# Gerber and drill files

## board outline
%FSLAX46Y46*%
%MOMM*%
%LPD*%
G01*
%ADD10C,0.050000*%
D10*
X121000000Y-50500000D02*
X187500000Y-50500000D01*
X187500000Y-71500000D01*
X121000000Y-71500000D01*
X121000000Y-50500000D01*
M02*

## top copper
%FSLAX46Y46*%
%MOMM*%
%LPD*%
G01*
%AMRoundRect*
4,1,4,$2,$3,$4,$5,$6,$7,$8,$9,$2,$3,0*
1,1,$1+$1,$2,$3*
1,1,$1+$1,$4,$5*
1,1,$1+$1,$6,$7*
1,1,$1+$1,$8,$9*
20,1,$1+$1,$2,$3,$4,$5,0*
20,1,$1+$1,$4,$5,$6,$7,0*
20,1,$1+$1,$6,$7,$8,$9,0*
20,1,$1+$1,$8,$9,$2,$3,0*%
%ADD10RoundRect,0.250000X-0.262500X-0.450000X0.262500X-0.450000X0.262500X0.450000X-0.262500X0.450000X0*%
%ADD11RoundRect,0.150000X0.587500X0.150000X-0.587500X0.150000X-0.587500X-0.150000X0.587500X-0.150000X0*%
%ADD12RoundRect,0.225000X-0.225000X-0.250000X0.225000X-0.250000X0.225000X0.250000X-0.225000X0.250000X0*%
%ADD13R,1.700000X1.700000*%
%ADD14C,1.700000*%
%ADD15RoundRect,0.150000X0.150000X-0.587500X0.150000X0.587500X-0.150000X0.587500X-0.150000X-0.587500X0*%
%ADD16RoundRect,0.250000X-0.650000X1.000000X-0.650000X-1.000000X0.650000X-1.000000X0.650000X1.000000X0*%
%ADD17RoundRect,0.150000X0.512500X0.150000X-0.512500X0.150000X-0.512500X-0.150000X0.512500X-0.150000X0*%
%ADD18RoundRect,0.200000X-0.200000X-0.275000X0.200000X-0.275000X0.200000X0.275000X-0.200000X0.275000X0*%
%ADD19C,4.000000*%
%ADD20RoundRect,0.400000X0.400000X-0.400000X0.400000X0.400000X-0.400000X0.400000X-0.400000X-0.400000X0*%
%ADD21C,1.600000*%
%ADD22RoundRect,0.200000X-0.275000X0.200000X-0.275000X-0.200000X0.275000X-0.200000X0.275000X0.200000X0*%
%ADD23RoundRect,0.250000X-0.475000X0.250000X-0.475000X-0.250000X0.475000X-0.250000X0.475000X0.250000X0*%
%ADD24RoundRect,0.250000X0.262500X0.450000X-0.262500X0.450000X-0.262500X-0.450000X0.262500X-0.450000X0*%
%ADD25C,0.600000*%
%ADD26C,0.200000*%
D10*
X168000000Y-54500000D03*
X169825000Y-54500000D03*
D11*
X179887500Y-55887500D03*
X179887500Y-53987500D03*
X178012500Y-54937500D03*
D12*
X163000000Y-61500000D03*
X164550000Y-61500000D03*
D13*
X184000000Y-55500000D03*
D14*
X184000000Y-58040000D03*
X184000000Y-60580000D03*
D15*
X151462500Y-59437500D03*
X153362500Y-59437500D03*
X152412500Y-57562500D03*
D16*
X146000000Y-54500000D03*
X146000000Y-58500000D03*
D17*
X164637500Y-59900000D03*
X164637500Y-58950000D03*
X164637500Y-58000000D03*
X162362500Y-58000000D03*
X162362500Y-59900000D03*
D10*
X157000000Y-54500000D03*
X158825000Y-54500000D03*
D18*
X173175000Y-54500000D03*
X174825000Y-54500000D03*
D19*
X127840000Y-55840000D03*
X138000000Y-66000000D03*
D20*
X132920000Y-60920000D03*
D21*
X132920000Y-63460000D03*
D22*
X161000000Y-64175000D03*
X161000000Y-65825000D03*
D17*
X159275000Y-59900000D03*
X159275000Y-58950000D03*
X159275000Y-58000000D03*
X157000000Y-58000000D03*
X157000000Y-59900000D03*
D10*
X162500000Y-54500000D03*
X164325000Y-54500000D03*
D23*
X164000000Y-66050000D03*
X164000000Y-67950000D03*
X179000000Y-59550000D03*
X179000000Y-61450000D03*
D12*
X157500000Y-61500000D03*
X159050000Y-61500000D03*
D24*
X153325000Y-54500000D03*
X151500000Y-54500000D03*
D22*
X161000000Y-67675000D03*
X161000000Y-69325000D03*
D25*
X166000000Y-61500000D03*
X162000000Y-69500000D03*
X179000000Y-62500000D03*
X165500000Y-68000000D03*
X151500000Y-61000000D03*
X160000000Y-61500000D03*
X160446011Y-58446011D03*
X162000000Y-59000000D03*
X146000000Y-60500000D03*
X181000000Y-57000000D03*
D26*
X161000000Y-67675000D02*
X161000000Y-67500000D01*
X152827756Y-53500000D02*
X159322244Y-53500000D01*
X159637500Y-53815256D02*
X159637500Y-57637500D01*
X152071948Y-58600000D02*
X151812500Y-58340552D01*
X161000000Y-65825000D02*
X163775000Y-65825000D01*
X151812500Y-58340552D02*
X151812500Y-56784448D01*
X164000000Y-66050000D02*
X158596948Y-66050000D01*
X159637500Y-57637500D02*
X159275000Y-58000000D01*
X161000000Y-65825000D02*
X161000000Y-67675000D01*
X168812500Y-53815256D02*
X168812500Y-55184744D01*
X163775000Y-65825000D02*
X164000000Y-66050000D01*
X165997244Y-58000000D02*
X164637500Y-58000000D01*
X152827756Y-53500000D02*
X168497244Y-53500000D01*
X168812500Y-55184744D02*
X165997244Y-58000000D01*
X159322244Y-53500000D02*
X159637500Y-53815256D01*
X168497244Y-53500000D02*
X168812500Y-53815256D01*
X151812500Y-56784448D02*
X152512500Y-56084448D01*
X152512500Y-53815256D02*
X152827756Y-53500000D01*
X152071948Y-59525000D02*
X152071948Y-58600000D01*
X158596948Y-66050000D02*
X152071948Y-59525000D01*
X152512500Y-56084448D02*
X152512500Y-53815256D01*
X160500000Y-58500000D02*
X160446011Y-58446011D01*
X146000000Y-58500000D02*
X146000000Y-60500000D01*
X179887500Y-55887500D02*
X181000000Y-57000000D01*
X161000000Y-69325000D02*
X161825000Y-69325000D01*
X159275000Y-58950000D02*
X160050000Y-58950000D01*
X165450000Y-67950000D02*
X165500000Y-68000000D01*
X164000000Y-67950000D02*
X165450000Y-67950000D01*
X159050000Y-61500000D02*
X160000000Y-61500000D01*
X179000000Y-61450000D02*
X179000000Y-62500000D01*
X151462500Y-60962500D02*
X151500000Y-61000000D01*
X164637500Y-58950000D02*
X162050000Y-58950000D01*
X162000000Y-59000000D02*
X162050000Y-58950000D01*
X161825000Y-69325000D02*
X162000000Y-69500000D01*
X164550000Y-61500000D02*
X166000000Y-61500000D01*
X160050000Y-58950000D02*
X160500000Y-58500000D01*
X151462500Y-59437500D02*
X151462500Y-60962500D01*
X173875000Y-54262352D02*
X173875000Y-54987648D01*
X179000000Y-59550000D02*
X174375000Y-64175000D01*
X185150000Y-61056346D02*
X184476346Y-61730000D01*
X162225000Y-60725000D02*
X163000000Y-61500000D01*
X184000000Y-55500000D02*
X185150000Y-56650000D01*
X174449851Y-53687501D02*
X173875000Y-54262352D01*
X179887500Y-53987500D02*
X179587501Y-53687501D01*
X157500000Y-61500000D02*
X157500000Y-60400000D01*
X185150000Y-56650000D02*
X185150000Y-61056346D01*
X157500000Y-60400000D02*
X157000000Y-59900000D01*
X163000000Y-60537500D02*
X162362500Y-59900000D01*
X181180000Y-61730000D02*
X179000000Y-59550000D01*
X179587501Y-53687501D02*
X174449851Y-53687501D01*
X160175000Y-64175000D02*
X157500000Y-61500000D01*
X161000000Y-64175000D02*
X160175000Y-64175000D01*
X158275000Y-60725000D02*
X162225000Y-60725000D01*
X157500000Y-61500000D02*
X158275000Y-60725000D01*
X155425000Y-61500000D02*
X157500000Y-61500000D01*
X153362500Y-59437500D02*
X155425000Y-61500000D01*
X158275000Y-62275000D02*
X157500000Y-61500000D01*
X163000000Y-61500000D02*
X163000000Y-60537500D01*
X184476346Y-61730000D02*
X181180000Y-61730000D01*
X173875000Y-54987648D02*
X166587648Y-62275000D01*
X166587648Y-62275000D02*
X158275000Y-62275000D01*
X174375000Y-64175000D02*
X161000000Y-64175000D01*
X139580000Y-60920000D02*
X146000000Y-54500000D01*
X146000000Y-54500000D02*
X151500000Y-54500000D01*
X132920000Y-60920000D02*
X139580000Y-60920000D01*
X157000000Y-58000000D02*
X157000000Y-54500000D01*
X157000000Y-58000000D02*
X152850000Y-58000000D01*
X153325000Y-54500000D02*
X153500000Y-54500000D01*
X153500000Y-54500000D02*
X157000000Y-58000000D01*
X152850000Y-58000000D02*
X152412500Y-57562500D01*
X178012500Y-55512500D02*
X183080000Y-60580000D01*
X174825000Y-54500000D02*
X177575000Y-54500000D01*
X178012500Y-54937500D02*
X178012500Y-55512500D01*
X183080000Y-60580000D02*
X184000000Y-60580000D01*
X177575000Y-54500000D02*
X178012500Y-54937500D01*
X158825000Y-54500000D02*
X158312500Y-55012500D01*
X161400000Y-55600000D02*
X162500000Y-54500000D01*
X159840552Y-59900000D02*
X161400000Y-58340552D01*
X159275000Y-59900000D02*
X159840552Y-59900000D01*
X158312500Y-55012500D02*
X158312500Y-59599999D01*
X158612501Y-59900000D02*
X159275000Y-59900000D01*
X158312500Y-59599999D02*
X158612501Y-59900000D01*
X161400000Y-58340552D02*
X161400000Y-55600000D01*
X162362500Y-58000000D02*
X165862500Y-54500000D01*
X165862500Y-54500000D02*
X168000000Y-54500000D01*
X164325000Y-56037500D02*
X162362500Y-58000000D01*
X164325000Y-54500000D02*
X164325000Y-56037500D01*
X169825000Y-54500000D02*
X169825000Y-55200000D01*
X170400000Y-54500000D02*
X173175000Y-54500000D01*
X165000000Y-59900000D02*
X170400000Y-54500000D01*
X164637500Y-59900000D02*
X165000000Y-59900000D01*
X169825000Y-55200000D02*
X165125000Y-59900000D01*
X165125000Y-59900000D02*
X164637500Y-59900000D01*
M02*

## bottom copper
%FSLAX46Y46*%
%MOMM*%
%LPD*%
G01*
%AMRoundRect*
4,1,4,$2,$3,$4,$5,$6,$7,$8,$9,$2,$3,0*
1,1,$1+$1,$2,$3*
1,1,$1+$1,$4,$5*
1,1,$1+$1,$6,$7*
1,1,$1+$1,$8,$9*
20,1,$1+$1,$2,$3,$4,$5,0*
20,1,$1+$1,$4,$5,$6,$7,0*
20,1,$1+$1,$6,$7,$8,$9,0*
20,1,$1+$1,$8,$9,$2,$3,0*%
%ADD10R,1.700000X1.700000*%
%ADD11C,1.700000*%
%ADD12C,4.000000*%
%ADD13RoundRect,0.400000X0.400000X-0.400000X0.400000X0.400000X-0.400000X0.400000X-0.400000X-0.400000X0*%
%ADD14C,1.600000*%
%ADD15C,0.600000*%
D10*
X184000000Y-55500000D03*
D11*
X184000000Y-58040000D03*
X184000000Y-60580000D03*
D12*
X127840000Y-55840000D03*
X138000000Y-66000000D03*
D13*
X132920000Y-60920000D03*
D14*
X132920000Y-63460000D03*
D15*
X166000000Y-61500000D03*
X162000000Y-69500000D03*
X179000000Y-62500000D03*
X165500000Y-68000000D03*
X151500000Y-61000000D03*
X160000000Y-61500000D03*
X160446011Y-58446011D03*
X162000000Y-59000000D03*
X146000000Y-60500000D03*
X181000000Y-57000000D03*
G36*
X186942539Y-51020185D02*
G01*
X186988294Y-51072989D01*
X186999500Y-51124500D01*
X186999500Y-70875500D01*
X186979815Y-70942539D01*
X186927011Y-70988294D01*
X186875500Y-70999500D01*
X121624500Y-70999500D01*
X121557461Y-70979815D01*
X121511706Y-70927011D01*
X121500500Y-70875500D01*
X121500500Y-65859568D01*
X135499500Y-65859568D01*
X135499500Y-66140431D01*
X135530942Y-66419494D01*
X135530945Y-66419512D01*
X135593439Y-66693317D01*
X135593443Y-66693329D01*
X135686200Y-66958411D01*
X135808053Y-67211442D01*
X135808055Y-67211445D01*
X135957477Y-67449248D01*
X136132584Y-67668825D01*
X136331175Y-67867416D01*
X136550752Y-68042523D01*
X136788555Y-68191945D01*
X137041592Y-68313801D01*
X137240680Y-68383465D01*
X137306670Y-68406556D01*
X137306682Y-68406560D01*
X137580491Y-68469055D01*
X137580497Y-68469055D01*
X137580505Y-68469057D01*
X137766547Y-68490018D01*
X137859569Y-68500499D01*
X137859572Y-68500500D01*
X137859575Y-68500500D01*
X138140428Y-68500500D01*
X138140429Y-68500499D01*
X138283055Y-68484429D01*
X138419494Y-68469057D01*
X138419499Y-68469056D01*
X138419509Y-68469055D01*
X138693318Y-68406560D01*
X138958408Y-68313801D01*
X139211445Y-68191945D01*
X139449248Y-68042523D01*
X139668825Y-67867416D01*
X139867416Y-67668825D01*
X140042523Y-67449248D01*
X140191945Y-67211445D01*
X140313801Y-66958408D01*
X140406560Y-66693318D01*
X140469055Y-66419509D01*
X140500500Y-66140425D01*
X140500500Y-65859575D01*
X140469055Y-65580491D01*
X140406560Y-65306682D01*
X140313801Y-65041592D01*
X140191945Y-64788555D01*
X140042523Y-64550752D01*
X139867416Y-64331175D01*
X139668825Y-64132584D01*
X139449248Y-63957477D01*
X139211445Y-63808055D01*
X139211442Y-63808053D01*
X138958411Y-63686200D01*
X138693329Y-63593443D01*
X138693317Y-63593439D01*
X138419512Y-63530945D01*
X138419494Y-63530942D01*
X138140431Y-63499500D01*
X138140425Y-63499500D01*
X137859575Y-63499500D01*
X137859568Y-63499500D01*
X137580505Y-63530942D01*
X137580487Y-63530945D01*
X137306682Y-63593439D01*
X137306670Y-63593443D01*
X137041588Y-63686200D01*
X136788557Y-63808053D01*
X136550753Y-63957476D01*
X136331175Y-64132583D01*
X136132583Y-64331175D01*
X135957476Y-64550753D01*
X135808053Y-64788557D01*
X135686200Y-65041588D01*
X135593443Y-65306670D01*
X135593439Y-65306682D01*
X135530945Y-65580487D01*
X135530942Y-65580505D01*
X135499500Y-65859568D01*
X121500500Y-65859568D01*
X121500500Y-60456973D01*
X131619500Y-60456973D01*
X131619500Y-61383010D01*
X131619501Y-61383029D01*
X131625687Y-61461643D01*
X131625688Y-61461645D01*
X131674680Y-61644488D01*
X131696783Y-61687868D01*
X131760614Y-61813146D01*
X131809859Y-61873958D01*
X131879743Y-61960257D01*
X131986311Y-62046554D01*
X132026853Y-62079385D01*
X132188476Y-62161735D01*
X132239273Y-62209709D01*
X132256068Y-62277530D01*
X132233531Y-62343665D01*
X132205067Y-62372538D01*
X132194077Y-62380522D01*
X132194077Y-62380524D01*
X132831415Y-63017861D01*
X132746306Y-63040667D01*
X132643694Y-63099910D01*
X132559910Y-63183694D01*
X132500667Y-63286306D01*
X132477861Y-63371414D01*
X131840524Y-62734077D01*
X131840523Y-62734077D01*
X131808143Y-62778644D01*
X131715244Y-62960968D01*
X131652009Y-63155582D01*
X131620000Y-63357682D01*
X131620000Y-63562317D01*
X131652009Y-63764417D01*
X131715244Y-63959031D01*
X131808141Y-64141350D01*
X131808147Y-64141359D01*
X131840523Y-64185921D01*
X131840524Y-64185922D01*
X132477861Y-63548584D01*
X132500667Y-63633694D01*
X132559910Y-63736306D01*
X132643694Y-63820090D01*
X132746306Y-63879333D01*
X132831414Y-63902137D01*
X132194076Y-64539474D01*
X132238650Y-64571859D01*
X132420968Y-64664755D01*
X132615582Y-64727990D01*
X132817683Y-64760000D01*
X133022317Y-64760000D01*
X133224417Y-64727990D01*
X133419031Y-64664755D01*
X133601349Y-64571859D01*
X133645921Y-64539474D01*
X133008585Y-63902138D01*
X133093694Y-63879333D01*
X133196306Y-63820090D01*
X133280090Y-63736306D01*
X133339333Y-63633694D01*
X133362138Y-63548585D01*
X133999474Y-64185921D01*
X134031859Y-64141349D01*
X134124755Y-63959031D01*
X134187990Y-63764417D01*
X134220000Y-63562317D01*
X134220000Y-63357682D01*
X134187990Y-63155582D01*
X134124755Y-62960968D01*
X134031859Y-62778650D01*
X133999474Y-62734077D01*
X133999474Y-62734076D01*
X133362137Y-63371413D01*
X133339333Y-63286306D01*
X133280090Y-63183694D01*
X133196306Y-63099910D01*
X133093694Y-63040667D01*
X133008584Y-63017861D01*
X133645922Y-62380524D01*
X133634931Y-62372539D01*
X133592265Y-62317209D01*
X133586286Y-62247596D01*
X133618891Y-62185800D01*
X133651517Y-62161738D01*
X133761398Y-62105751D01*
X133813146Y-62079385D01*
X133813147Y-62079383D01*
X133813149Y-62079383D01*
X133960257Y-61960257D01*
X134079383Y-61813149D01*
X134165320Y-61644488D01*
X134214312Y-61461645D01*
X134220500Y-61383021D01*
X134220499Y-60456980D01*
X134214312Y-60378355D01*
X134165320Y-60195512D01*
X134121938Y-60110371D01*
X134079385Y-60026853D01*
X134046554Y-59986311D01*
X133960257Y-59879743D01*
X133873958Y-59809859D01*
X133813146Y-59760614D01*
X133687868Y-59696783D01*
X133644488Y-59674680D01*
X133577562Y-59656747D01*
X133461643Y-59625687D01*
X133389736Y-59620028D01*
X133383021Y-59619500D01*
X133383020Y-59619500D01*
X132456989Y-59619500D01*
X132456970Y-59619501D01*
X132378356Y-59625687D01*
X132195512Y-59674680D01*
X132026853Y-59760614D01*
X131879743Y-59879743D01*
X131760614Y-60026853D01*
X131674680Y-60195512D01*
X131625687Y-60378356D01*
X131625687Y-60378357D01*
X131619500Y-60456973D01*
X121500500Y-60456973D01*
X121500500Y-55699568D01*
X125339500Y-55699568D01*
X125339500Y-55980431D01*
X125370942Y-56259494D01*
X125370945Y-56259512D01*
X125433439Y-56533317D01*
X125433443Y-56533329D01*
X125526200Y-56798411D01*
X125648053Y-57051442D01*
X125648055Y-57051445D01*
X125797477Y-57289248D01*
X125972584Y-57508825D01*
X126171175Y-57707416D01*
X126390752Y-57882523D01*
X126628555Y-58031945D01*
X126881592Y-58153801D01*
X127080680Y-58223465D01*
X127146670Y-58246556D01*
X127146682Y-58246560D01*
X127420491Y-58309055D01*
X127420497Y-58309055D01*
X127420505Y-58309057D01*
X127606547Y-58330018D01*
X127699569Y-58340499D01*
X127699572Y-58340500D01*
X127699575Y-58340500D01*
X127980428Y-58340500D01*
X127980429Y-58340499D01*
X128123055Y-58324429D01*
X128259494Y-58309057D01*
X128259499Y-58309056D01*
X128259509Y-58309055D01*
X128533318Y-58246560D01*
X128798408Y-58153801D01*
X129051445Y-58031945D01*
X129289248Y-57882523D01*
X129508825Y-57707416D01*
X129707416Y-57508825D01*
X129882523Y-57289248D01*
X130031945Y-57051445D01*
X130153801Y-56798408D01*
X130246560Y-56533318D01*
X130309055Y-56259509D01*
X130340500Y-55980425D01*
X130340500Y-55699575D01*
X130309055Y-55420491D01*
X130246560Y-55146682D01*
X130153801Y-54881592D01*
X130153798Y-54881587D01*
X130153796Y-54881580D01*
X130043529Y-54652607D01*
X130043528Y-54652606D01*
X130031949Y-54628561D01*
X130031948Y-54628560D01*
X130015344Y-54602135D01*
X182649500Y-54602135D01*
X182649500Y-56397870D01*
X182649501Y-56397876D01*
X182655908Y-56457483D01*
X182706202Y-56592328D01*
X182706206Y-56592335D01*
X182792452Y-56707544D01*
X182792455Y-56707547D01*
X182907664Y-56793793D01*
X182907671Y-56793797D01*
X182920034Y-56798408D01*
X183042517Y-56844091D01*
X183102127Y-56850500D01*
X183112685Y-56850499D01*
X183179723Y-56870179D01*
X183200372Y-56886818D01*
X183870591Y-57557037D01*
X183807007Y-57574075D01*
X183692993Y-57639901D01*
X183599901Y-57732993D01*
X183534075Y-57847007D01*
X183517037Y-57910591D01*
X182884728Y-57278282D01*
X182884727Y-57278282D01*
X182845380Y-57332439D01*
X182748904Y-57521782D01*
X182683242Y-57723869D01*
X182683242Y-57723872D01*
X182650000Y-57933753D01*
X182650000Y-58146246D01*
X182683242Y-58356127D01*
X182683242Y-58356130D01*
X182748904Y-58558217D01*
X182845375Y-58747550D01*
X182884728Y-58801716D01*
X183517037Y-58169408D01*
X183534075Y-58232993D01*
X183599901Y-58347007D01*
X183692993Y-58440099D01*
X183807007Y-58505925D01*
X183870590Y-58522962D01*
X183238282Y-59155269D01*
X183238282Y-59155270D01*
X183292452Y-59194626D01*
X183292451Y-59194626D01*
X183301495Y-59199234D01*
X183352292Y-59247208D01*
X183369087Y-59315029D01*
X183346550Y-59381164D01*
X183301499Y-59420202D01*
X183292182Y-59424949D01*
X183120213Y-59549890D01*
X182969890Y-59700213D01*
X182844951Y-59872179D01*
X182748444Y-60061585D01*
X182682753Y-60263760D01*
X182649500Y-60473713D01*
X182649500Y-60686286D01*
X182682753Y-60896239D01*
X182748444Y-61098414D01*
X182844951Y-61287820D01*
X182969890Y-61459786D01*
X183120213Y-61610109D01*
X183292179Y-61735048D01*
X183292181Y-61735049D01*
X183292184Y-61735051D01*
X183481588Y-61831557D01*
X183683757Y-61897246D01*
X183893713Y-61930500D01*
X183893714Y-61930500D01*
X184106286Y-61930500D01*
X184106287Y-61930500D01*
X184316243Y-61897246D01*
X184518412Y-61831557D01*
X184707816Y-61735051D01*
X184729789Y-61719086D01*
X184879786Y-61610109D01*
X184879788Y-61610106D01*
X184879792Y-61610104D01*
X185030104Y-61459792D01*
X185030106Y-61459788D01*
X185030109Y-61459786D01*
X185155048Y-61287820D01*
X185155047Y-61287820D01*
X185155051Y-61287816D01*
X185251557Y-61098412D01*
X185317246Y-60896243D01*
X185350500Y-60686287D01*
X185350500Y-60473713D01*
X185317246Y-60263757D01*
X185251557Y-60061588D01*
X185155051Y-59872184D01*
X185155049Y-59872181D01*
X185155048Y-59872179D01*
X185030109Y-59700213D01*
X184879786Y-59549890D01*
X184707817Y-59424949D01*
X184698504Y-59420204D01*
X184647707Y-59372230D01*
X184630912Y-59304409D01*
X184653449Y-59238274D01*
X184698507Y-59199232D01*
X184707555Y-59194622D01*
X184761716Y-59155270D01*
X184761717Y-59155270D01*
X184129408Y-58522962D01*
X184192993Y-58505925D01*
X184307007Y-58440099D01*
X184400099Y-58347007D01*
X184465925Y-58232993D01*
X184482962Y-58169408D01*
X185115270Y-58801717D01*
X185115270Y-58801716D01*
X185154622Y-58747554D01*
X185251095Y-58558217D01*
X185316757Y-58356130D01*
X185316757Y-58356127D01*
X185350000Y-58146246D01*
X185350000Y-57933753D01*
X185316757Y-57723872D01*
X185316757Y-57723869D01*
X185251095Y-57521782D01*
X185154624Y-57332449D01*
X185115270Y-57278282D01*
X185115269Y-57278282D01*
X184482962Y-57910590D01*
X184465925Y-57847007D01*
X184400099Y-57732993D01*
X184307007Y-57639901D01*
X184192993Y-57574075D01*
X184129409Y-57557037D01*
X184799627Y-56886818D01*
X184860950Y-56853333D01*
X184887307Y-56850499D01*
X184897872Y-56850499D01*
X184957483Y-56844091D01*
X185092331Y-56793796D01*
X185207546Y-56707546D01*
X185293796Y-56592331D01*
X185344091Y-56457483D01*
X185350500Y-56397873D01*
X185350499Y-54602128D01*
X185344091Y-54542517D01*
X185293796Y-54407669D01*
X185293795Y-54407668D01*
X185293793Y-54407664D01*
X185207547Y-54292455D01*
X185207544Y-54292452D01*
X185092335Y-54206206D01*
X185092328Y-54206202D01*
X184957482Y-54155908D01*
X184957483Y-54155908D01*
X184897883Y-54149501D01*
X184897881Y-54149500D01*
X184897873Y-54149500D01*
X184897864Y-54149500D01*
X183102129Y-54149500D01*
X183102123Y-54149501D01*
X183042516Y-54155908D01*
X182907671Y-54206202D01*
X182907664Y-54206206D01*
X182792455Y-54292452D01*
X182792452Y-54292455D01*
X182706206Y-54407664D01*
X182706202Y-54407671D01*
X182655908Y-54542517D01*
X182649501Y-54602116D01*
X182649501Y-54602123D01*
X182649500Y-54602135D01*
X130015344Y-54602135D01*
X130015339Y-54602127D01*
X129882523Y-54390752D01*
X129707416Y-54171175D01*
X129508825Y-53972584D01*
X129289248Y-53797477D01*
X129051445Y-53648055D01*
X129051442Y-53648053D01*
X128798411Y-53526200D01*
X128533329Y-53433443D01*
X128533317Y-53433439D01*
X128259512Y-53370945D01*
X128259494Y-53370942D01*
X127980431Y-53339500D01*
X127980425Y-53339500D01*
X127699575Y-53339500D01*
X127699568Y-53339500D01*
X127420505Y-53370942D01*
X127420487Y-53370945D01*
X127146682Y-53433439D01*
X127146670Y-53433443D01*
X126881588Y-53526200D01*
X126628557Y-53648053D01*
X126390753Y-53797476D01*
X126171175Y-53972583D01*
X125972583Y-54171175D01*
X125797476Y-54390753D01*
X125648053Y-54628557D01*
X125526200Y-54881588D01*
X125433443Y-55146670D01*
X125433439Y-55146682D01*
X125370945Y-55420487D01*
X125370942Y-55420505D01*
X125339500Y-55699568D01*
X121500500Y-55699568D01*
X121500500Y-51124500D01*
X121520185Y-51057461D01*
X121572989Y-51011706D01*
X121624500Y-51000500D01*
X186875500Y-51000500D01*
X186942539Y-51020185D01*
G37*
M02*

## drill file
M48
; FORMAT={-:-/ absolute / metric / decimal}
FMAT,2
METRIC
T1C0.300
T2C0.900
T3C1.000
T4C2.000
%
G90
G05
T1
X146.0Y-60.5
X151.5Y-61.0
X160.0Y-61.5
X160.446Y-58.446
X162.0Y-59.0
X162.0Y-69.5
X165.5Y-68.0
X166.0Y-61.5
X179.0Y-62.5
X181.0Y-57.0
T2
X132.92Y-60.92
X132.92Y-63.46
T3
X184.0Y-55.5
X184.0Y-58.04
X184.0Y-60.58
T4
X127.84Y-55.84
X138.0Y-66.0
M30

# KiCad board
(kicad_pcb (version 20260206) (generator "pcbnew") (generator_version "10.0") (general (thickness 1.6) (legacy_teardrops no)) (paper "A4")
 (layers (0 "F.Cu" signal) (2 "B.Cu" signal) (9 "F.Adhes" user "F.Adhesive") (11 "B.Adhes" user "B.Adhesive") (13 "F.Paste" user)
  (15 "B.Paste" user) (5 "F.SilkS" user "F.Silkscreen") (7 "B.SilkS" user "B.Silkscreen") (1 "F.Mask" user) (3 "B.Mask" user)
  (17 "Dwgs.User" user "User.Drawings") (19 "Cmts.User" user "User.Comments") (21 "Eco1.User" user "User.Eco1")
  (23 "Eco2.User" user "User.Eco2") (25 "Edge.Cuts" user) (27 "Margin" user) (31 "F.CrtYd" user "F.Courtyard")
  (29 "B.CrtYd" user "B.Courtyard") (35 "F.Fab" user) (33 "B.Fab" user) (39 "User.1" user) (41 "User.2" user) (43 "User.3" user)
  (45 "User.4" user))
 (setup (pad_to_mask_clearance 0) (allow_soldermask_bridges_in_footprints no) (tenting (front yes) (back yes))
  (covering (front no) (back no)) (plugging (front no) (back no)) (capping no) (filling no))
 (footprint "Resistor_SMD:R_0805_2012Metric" (layer "F.Cu") (at 168.9125 54.5)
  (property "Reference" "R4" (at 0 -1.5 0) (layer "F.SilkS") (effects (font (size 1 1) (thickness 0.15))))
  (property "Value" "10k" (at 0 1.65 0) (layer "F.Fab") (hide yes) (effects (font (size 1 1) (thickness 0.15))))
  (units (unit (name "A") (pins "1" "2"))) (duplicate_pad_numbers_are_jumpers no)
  (pad "1" smd roundrect (at -0.9125 0) (size 1.025 1.4) (layers "F.Cu" "F.Mask" "F.Paste") (roundrect_rratio 0.243902) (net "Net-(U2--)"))
  (pad "2" smd roundrect (at 0.9125 0) (size 1.025 1.4) (layers "F.Cu" "F.Mask" "F.Paste") (roundrect_rratio 0.243902) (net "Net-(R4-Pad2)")))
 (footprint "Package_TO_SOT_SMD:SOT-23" (layer "F.Cu") (at 178.95 54.9375 180)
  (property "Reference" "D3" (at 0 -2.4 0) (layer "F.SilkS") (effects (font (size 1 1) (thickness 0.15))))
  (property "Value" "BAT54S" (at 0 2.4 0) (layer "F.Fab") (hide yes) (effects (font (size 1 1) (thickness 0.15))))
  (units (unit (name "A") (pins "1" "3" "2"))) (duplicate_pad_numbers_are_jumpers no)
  (pad "1" smd roundrect (at -0.9375 -0.95 180) (size 1.475 0.6) (layers "F.Cu" "F.Mask" "F.Paste") (roundrect_rratio 0.25) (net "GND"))
  (pad "2" smd roundrect (at -0.9375 0.95 180) (size 1.475 0.6) (layers "F.Cu" "F.Mask" "F.Paste") (roundrect_rratio 0.25)
   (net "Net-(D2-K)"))
  (pad "3" smd roundrect (at 0.9375 0 180) (size 1.475 0.6) (layers "F.Cu" "F.Mask" "F.Paste") (roundrect_rratio 0.25) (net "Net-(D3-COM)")))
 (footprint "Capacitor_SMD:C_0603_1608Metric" (layer "F.Cu") (at 163.775 61.5)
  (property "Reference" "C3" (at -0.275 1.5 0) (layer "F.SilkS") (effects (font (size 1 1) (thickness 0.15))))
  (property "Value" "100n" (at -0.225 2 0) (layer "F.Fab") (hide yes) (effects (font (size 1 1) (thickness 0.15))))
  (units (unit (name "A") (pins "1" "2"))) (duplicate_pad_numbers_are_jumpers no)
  (pad "1" smd roundrect (at -0.775 0) (size 0.9 0.95) (layers "F.Cu" "F.Mask" "F.Paste") (roundrect_rratio 0.25) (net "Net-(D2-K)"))
  (pad "2" smd roundrect (at 0.775 0) (size 0.9 0.95) (layers "F.Cu" "F.Mask" "F.Paste") (roundrect_rratio 0.25) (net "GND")))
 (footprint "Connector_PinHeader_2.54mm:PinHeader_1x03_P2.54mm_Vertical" (layer "F.Cu") (at 184 55.5)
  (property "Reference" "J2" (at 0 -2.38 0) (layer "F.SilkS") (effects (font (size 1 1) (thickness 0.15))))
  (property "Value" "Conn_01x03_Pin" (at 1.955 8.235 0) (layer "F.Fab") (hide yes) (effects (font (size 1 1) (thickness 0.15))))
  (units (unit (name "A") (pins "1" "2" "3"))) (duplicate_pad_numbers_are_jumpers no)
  (pad "1" thru_hole rect (at 0 0) (size 1.7 1.7) (drill 1) (layers "*.Cu" "*.Mask") (remove_unused_layers no) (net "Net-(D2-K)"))
  (pad "2" thru_hole circle (at 0 2.54) (size 1.7 1.7) (drill 1) (layers "*.Cu" "*.Mask") (remove_unused_layers no) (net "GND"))
  (pad "3" thru_hole circle (at 0 5.08) (size 1.7 1.7) (drill 1) (layers "*.Cu" "*.Mask") (remove_unused_layers no) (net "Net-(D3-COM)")))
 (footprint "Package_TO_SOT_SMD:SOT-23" (layer "F.Cu") (at 152.4125 58.5 90)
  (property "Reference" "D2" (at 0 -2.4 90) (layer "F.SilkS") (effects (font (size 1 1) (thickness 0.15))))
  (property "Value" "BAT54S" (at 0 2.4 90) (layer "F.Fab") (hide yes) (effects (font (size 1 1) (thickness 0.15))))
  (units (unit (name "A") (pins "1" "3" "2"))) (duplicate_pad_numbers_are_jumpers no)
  (pad "1" smd roundrect (at -0.9375 -0.95 90) (size 1.475 0.6) (layers "F.Cu" "F.Mask" "F.Paste") (roundrect_rratio 0.25) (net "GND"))
  (pad "2" smd roundrect (at -0.9375 0.95 90) (size 1.475 0.6) (layers "F.Cu" "F.Mask" "F.Paste") (roundrect_rratio 0.25) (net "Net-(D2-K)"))
  (pad "3" smd roundrect (at 0.9375 0 90) (size 1.475 0.6) (layers "F.Cu" "F.Mask" "F.Paste") (roundrect_rratio 0.25) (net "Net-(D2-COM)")))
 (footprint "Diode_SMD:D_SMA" (layer "F.Cu") (at 146 56.5 -90)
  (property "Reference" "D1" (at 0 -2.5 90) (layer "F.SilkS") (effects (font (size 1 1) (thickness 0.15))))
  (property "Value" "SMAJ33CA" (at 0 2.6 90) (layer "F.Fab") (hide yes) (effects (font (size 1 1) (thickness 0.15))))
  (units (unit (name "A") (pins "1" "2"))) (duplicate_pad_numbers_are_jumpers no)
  (pad "1" smd roundrect (at -2 0 270) (size 2.5 1.8) (layers "F.Cu" "F.Mask" "F.Paste") (roundrect_rratio 0.1388888889) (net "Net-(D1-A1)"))
  (pad "2" smd roundrect (at 2 0 270) (size 2.5 1.8) (layers "F.Cu" "F.Mask" "F.Paste") (roundrect_rratio 0.1388888889) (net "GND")))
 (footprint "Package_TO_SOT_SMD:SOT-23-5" (layer "F.Cu") (at 163.5 58.95 180)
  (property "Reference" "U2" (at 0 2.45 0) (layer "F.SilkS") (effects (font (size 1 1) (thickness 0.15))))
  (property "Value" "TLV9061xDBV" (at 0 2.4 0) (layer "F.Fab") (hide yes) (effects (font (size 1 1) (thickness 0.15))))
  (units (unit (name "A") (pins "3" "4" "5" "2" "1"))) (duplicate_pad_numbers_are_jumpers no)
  (pad "1" smd roundrect (at -1.1375 -0.95 180) (size 1.325 0.6) (layers "F.Cu" "F.Mask" "F.Paste") (roundrect_rratio 0.25)
   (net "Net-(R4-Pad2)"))
  (pad "2" smd roundrect (at -1.1375 0 180) (size 1.325 0.6) (layers "F.Cu" "F.Mask" "F.Paste") (roundrect_rratio 0.25) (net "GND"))
  (pad "3" smd roundrect (at -1.1375 0.95 180) (size 1.325 0.6) (layers "F.Cu" "F.Mask" "F.Paste") (roundrect_rratio 0.25)
   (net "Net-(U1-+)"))
  (pad "4" smd roundrect (at 1.1375 0.95 180) (size 1.325 0.6) (layers "F.Cu" "F.Mask" "F.Paste") (roundrect_rratio 0.25) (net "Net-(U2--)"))
  (pad "5" smd roundrect (at 1.1375 -0.95 180) (size 1.325 0.6) (layers "F.Cu" "F.Mask" "F.Paste") (roundrect_rratio 0.25)
   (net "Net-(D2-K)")))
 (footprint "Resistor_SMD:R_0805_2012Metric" (layer "F.Cu") (at 157.9125 54.5)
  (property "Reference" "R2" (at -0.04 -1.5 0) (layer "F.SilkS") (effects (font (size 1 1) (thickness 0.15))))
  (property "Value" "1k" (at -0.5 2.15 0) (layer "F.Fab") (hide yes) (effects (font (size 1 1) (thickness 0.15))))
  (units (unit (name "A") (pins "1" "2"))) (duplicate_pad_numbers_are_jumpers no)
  (pad "1" smd roundrect (at -0.9125 0) (size 1.025 1.4) (layers "F.Cu" "F.Mask" "F.Paste") (roundrect_rratio 0.243902) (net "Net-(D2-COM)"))
  (pad "2" smd roundrect (at 0.9125 0) (size 1.025 1.4) (layers "F.Cu" "F.Mask" "F.Paste") (roundrect_rratio 0.243902) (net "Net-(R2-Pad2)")))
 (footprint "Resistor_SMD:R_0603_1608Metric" (layer "F.Cu") (at 174 54.5)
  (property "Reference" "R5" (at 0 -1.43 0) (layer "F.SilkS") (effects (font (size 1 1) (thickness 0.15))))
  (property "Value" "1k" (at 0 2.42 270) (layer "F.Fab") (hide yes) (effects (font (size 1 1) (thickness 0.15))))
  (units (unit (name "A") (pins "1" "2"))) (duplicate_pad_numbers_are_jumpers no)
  (pad "1" smd roundrect (at -0.825 0) (size 0.8 0.95) (layers "F.Cu" "F.Mask" "F.Paste") (roundrect_rratio 0.25) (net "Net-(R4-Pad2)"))
  (pad "2" smd roundrect (at 0.825 0) (size 0.8 0.95) (layers "F.Cu" "F.Mask" "F.Paste") (roundrect_rratio 0.25) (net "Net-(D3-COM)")))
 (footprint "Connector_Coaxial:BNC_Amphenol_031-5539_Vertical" (layer "F.Cu") (at 132.92 60.92 -90)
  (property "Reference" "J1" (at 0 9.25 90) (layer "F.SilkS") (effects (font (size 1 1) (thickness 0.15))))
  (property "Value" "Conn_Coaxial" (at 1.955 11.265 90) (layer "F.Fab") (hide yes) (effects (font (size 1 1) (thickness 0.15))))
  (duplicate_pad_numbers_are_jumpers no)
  (pad "" thru_hole circle (at -5.08 5.08 90) (size 4 4) (drill 2) (layers "*.Cu" "*.Mask") (remove_unused_layers no))
  (pad "" thru_hole circle (at 5.08 -5.08 90) (size 4 4) (drill 2) (layers "*.Cu" "*.Mask") (remove_unused_layers no))
  (pad "1" thru_hole roundrect (at 0 0 90) (size 1.6 1.6) (drill 0.9) (layers "*.Cu" "*.Mask") (remove_unused_layers no)
   (roundrect_rratio 0.25) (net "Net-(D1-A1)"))
  (pad "2" thru_hole circle (at 2.54 0 90) (size 1.6 1.6) (drill 0.9) (layers "*.Cu" "*.Mask") (remove_unused_layers no) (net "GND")))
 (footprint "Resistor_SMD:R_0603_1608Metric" (layer "F.Cu") (at 161 65 -90)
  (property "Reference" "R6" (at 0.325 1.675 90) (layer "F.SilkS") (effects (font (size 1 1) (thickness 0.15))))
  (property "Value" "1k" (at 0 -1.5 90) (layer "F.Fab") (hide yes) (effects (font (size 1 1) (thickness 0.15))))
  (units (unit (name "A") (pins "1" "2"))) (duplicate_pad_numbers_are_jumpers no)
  (pad "1" smd roundrect (at -0.825 0 270) (size 0.8 0.95) (layers "F.Cu" "F.Mask" "F.Paste") (roundrect_rratio 0.25) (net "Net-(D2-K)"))
  (pad "2" smd roundrect (at 0.825 0 270) (size 0.8 0.95) (layers "F.Cu" "F.Mask" "F.Paste") (roundrect_rratio 0.25) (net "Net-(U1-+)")))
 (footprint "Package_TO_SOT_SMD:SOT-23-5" (layer "F.Cu") (at 158.1375 58.95 180)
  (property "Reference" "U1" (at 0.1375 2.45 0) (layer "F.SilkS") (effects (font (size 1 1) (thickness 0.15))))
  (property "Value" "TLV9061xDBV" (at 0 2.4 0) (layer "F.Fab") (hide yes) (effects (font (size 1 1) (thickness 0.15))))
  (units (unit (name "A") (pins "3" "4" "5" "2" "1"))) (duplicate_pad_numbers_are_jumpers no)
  (pad "1" smd roundrect (at -1.1375 -0.95 180) (size 1.325 0.6) (layers "F.Cu" "F.Mask" "F.Paste") (roundrect_rratio 0.25)
   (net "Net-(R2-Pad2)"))
  (pad "2" smd roundrect (at -1.1375 0 180) (size 1.325 0.6) (layers "F.Cu" "F.Mask" "F.Paste") (roundrect_rratio 0.25) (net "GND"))
  (pad "3" smd roundrect (at -1.1375 0.95 180) (size 1.325 0.6) (layers "F.Cu" "F.Mask" "F.Paste") (roundrect_rratio 0.25)
   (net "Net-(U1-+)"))
  (pad "4" smd roundrect (at 1.1375 0.95 180) (size 1.325 0.6) (layers "F.Cu" "F.Mask" "F.Paste") (roundrect_rratio 0.25)
   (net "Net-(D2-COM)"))
  (pad "5" smd roundrect (at 1.1375 -0.95 180) (size 1.325 0.6) (layers "F.Cu" "F.Mask" "F.Paste") (roundrect_rratio 0.25)
   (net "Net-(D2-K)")))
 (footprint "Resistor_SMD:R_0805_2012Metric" (layer "F.Cu") (at 163.4125 54.5)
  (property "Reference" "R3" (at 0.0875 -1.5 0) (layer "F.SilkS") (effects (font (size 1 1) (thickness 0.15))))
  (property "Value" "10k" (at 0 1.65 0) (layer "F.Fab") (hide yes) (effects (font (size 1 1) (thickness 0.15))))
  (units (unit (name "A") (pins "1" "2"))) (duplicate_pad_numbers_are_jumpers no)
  (pad "1" smd roundrect (at -0.9125 0) (size 1.025 1.4) (layers "F.Cu" "F.Mask" "F.Paste") (roundrect_rratio 0.243902)
   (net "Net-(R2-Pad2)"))
  (pad "2" smd roundrect (at 0.9125 0) (size 1.025 1.4) (layers "F.Cu" "F.Mask" "F.Paste") (roundrect_rratio 0.243902) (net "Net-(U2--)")))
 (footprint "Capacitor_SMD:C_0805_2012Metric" (layer "F.Cu") (at 164 67 -90)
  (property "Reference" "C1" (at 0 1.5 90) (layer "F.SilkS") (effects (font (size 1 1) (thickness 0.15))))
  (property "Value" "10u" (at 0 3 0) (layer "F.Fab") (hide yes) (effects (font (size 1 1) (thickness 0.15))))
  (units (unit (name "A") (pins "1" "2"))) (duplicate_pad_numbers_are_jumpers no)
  (pad "1" smd roundrect (at -0.95 0 270) (size 1 1.45) (layers "F.Cu" "F.Mask" "F.Paste") (roundrect_rratio 0.25) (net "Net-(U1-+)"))
  (pad "2" smd roundrect (at 0.95 0 270) (size 1 1.45) (layers "F.Cu" "F.Mask" "F.Paste") (roundrect_rratio 0.25) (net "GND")))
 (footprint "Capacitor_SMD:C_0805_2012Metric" (layer "F.Cu") (at 179 60.5 -90)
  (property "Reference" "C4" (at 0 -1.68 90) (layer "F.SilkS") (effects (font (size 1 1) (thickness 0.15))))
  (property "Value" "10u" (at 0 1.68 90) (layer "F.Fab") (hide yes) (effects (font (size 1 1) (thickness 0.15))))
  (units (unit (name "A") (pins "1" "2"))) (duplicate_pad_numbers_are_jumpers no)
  (pad "1" smd roundrect (at -0.95 0 270) (size 1 1.45) (layers "F.Cu" "F.Mask" "F.Paste") (roundrect_rratio 0.25) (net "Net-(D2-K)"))
  (pad "2" smd roundrect (at 0.95 0 270) (size 1 1.45) (layers "F.Cu" "F.Mask" "F.Paste") (roundrect_rratio 0.25) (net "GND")))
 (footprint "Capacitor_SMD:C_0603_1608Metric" (layer "F.Cu") (at 158.275 61.5)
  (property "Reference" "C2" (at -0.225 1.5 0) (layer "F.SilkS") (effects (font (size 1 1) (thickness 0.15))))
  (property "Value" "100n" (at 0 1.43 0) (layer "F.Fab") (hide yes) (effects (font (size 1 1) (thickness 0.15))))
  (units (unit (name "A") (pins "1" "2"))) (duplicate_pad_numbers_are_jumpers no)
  (pad "1" smd roundrect (at -0.775 0) (size 0.9 0.95) (layers "F.Cu" "F.Mask" "F.Paste") (roundrect_rratio 0.25) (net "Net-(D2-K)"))
  (pad "2" smd roundrect (at 0.775 0) (size 0.9 0.95) (layers "F.Cu" "F.Mask" "F.Paste") (roundrect_rratio 0.25) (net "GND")))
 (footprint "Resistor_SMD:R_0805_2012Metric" (layer "F.Cu") (at 152.4125 54.5 180)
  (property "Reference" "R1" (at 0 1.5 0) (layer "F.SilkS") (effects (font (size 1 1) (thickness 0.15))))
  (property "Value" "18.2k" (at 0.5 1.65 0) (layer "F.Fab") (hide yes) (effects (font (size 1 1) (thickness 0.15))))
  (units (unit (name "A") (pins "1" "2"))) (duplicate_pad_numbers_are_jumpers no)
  (pad "1" smd roundrect (at -0.9125 0 180) (size 1.025 1.4) (layers "F.Cu" "F.Mask" "F.Paste") (roundrect_rratio 0.243902)
   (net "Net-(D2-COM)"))
  (pad "2" smd roundrect (at 0.9125 0 180) (size 1.025 1.4) (layers "F.Cu" "F.Mask" "F.Paste") (roundrect_rratio 0.243902)
   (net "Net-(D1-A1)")))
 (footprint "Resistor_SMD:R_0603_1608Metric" (layer "F.Cu") (at 161 68.5 -90)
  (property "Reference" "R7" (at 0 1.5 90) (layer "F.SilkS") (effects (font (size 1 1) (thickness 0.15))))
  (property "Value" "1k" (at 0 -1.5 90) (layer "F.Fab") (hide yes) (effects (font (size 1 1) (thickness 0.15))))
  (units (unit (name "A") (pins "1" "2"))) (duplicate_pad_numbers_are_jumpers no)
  (pad "1" smd roundrect (at -0.825 0 270) (size 0.8 0.95) (layers "F.Cu" "F.Mask" "F.Paste") (roundrect_rratio 0.25) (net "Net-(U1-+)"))
  (pad "2" smd roundrect (at 0.825 0 270) (size 0.8 0.95) (layers "F.Cu" "F.Mask" "F.Paste") (roundrect_rratio 0.25) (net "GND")))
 (gr_rect (start 121 50.5) (end 187.5 71.5) (stroke (width 0.05) (type solid)) (fill no) (layer "Edge.Cuts"))
 (segment (start 161 67.675) (end 161 67.5) (width 0.2) (layer "F.Cu") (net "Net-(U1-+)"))
 (segment (start 152.827756 53.5) (end 159.322244 53.5) (width 0.2) (layer "F.Cu") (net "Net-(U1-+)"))
 (segment (start 159.6375 53.815256) (end 159.6375 57.6375) (width 0.2) (layer "F.Cu") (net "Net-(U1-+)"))
 (segment (start 152.071948 58.6) (end 151.8125 58.340552) (width 0.2) (layer "F.Cu") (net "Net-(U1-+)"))
 (segment (start 161 65.825) (end 163.775 65.825) (width 0.2) (layer "F.Cu") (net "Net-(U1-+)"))
 (segment (start 151.8125 58.340552) (end 151.8125 56.784448) (width 0.2) (layer "F.Cu") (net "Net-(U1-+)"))
 (segment (start 164 66.05) (end 158.596948 66.05) (width 0.2) (layer "F.Cu") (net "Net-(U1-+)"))
 (segment (start 159.6375 57.6375) (end 159.275 58) (width 0.2) (layer "F.Cu") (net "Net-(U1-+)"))
 (segment (start 161 65.825) (end 161 67.675) (width 0.2) (layer "F.Cu") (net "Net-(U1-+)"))
 (segment (start 168.8125 53.815256) (end 168.8125 55.184744) (width 0.2) (layer "F.Cu") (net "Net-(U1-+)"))
 (segment (start 163.775 65.825) (end 164 66.05) (width 0.2) (layer "F.Cu") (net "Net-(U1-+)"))
 (segment (start 165.997244 58) (end 164.6375 58) (width 0.2) (layer "F.Cu") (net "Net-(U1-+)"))
 (segment (start 152.827756 53.5) (end 168.497244 53.5) (width 0.2) (layer "F.Cu") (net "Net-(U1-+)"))
 (segment (start 168.8125 55.184744) (end 165.997244 58) (width 0.2) (layer "F.Cu") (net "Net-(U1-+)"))
 (segment (start 159.322244 53.5) (end 159.6375 53.815256) (width 0.2) (layer "F.Cu") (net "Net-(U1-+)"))
 (segment (start 168.497244 53.5) (end 168.8125 53.815256) (width 0.2) (layer "F.Cu") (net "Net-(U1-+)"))
 (segment (start 151.8125 56.784448) (end 152.5125 56.084448) (width 0.2) (layer "F.Cu") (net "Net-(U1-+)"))
 (segment (start 152.5125 53.815256) (end 152.827756 53.5) (width 0.2) (layer "F.Cu") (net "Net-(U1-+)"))
 (segment (start 152.071948 59.525) (end 152.071948 58.6) (width 0.2) (layer "F.Cu") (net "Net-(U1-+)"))
 (segment (start 158.596948 66.05) (end 152.071948 59.525) (width 0.2) (layer "F.Cu") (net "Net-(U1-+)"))
 (segment (start 152.5125 56.084448) (end 152.5125 53.815256) (width 0.2) (layer "F.Cu") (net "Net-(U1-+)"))
 (segment (start 160.5 58.5) (end 160.446011 58.446011) (width 0.2) (layer "F.Cu") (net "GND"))
 (segment (start 146 58.5) (end 146 60.5) (width 0.2) (layer "F.Cu") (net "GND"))
 (segment (start 179.8875 55.8875) (end 181 57) (width 0.2) (layer "F.Cu") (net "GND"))
 (segment (start 161 69.325) (end 161.825 69.325) (width 0.2) (layer "F.Cu") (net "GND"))
 (segment (start 159.275 58.95) (end 160.05 58.95) (width 0.2) (layer "F.Cu") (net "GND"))
 (segment (start 165.45 67.95) (end 165.5 68) (width 0.2) (layer "F.Cu") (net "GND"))
 (segment (start 164 67.95) (end 165.45 67.95) (width 0.2) (layer "F.Cu") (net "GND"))
 (segment (start 159.05 61.5) (end 160 61.5) (width 0.2) (layer "F.Cu") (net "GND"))
 (segment (start 179 61.45) (end 179 62.5) (width 0.2) (layer "F.Cu") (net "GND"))
 (segment (start 151.4625 60.9625) (end 151.5 61) (width 0.2) (layer "F.Cu") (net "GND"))
 (segment (start 164.6375 58.95) (end 162.05 58.95) (width 0.2) (layer "F.Cu") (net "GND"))
 (segment (start 162 59) (end 162.05 58.95) (width 0.2) (layer "F.Cu") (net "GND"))
 (segment (start 161.825 69.325) (end 162 69.5) (width 0.2) (layer "F.Cu") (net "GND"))
 (segment (start 164.55 61.5) (end 166 61.5) (width 0.2) (layer "F.Cu") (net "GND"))
 (segment (start 160.05 58.95) (end 160.5 58.5) (width 0.2) (layer "F.Cu") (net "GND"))
 (segment (start 151.4625 59.4375) (end 151.4625 60.9625) (width 0.2) (layer "F.Cu") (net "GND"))
 (via (at 166 61.5) (size 0.6) (drill 0.3) (layers "F.Cu" "B.Cu") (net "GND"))
 (via (at 162 69.5) (size 0.6) (drill 0.3) (layers "F.Cu" "B.Cu") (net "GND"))
 (via (at 179 62.5) (size 0.6) (drill 0.3) (layers "F.Cu" "B.Cu") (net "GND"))
 (via (at 165.5 68) (size 0.6) (drill 0.3) (layers "F.Cu" "B.Cu") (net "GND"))
 (via (at 151.5 61) (size 0.6) (drill 0.3) (layers "F.Cu" "B.Cu") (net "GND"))
 (via (at 160 61.5) (size 0.6) (drill 0.3) (layers "F.Cu" "B.Cu") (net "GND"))
 (via (at 160.446011 58.446011) (size 0.6) (drill 0.3) (layers "F.Cu" "B.Cu") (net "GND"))
 (via (at 162 59) (size 0.6) (drill 0.3) (layers "F.Cu" "B.Cu") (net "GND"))
 (via (at 146 60.5) (size 0.6) (drill 0.3) (layers "F.Cu" "B.Cu") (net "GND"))
 (via (at 181 57) (size 0.6) (drill 0.3) (layers "F.Cu" "B.Cu") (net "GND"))
 (segment (start 173.875 54.262352) (end 173.875 54.987648) (width 0.2) (layer "F.Cu") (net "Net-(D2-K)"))
 (segment (start 179 59.55) (end 174.375 64.175) (width 0.2) (layer "F.Cu") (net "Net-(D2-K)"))
 (segment (start 185.15 61.056346) (end 184.476346 61.73) (width 0.2) (layer "F.Cu") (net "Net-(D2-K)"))
 (segment (start 162.225 60.725) (end 163 61.5) (width 0.2) (layer "F.Cu") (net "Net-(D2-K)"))
 (segment (start 184 55.5) (end 185.15 56.65) (width 0.2) (layer "F.Cu") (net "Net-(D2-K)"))
 (segment (start 174.449851 53.687501) (end 173.875 54.262352) (width 0.2) (layer "F.Cu") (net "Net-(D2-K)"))
 (segment (start 179.8875 53.9875) (end 179.587501 53.687501) (width 0.2) (layer "F.Cu") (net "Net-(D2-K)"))
 (segment (start 157.5 61.5) (end 157.5 60.4) (width 0.2) (layer "F.Cu") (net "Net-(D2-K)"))
 (segment (start 185.15 56.65) (end 185.15 61.056346) (width 0.2) (layer "F.Cu") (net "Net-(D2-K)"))
 (segment (start 157.5 60.4) (end 157 59.9) (width 0.2) (layer "F.Cu") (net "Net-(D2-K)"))
 (segment (start 163 60.5375) (end 162.3625 59.9) (width 0.2) (layer "F.Cu") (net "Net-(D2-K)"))
 (segment (start 181.18 61.73) (end 179 59.55) (width 0.2) (layer "F.Cu") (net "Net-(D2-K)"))
 (segment (start 179.587501 53.687501) (end 174.449851 53.687501) (width 0.2) (layer "F.Cu") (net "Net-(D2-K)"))
 (segment (start 160.175 64.175) (end 157.5 61.5) (width 0.2) (layer "F.Cu") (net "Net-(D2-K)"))
 (segment (start 161 64.175) (end 160.175 64.175) (width 0.2) (layer "F.Cu") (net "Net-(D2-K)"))
 (segment (start 158.275 60.725) (end 162.225 60.725) (width 0.2) (layer "F.Cu") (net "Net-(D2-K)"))
 (segment (start 157.5 61.5) (end 158.275 60.725) (width 0.2) (layer "F.Cu") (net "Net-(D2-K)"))
 (segment (start 155.425 61.5) (end 157.5 61.5) (width 0.2) (layer "F.Cu") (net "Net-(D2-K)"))
 (segment (start 153.3625 59.4375) (end 155.425 61.5) (width 0.2) (layer "F.Cu") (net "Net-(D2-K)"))
 (segment (start 158.275 62.275) (end 157.5 61.5) (width 0.2) (layer "F.Cu") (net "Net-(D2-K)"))
 (segment (start 163 61.5) (end 163 60.5375) (width 0.2) (layer "F.Cu") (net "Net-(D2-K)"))
 (segment (start 184.476346 61.73) (end 181.18 61.73) (width 0.2) (layer "F.Cu") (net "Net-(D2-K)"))
 (segment (start 173.875 54.987648) (end 166.587648 62.275) (width 0.2) (layer "F.Cu") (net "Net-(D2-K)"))
 (segment (start 166.587648 62.275) (end 158.275 62.275) (width 0.2) (layer "F.Cu") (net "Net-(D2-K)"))
 (segment (start 174.375 64.175) (end 161 64.175) (width 0.2) (layer "F.Cu") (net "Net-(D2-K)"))
 (segment (start 139.58 60.92) (end 146 54.5) (width 0.2) (layer "F.Cu") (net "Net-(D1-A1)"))
 (segment (start 146 54.5) (end 151.5 54.5) (width 0.2) (layer "F.Cu") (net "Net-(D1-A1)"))
 (segment (start 132.92 60.92) (end 139.58 60.92) (width 0.2) (layer "F.Cu") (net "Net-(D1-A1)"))
 (segment (start 157 58) (end 157 54.5) (width 0.2) (layer "F.Cu") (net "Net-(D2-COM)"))
 (segment (start 157 58) (end 152.85 58) (width 0.2) (layer "F.Cu") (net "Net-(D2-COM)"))
 (segment (start 153.325 54.5) (end 153.5 54.5) (width 0.2) (layer "F.Cu") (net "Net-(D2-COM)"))
 (segment (start 153.5 54.5) (end 157 58) (width 0.2) (layer "F.Cu") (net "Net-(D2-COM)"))
 (segment (start 152.85 58) (end 152.4125 57.5625) (width 0.2) (layer "F.Cu") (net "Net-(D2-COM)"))
 (segment (start 178.0125 55.5125) (end 183.08 60.58) (width 0.2) (layer "F.Cu") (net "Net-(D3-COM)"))
 (segment (start 174.825 54.5) (end 177.575 54.5) (width 0.2) (layer "F.Cu") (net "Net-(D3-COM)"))
 (segment (start 178.0125 54.9375) (end 178.0125 55.5125) (width 0.2) (layer "F.Cu") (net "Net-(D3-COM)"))
 (segment (start 183.08 60.58) (end 184 60.58) (width 0.2) (layer "F.Cu") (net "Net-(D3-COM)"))
 (segment (start 177.575 54.5) (end 178.0125 54.9375) (width 0.2) (layer "F.Cu") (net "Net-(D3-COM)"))
 (segment (start 158.825 54.5) (end 158.3125 55.0125) (width 0.2) (layer "F.Cu") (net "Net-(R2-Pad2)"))
 (segment (start 161.4 55.6) (end 162.5 54.5) (width 0.2) (layer "F.Cu") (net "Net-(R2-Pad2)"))
 (segment (start 159.840552 59.9) (end 161.4 58.340552) (width 0.2) (layer "F.Cu") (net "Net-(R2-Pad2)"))
 (segment (start 159.275 59.9) (end 159.840552 59.9) (width 0.2) (layer "F.Cu") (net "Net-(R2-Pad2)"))
 (segment (start 158.3125 55.0125) (end 158.3125 59.599999) (width 0.2) (layer "F.Cu") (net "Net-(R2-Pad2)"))
 (segment (start 158.612501 59.9) (end 159.275 59.9) (width 0.2) (layer "F.Cu") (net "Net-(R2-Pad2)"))
 (segment (start 158.3125 59.599999) (end 158.612501 59.9) (width 0.2) (layer "F.Cu") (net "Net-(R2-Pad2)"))
 (segment (start 161.4 58.340552) (end 161.4 55.6) (width 0.2) (layer "F.Cu") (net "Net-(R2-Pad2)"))
 (segment (start 162.3625 58) (end 165.8625 54.5) (width 0.2) (layer "F.Cu") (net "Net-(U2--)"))
 (segment (start 165.8625 54.5) (end 168 54.5) (width 0.2) (layer "F.Cu") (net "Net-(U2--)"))
 (segment (start 164.325 56.0375) (end 162.3625 58) (width 0.2) (layer "F.Cu") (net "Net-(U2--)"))
 (segment (start 164.325 54.5) (end 164.325 56.0375) (width 0.2) (layer "F.Cu") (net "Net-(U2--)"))
 (segment (start 169.825 54.5) (end 169.825 55.2) (width 0.2) (layer "F.Cu") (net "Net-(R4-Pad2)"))
 (segment (start 170.4 54.5) (end 173.175 54.5) (width 0.2) (layer "F.Cu") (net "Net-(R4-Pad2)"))
 (segment (start 165 59.9) (end 170.4 54.5) (width 0.2) (layer "F.Cu") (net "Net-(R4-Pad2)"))
 (segment (start 164.6375 59.9) (end 165 59.9) (width 0.2) (layer "F.Cu") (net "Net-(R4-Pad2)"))
 (segment (start 169.825 55.2) (end 165.125 59.9) (width 0.2) (layer "F.Cu") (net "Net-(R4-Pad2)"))
 (segment (start 165.125 59.9) (end 164.6375 59.9) (width 0.2) (layer "F.Cu") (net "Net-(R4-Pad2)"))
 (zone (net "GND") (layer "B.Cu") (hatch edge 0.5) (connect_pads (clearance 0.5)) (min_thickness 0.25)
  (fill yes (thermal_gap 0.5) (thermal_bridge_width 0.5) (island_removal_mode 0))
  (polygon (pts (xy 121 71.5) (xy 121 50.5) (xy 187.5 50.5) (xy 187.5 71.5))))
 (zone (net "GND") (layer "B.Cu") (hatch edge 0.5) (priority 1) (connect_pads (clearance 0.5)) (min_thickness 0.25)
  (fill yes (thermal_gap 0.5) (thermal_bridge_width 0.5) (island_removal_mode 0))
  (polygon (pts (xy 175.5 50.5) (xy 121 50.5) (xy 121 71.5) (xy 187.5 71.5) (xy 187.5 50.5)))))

